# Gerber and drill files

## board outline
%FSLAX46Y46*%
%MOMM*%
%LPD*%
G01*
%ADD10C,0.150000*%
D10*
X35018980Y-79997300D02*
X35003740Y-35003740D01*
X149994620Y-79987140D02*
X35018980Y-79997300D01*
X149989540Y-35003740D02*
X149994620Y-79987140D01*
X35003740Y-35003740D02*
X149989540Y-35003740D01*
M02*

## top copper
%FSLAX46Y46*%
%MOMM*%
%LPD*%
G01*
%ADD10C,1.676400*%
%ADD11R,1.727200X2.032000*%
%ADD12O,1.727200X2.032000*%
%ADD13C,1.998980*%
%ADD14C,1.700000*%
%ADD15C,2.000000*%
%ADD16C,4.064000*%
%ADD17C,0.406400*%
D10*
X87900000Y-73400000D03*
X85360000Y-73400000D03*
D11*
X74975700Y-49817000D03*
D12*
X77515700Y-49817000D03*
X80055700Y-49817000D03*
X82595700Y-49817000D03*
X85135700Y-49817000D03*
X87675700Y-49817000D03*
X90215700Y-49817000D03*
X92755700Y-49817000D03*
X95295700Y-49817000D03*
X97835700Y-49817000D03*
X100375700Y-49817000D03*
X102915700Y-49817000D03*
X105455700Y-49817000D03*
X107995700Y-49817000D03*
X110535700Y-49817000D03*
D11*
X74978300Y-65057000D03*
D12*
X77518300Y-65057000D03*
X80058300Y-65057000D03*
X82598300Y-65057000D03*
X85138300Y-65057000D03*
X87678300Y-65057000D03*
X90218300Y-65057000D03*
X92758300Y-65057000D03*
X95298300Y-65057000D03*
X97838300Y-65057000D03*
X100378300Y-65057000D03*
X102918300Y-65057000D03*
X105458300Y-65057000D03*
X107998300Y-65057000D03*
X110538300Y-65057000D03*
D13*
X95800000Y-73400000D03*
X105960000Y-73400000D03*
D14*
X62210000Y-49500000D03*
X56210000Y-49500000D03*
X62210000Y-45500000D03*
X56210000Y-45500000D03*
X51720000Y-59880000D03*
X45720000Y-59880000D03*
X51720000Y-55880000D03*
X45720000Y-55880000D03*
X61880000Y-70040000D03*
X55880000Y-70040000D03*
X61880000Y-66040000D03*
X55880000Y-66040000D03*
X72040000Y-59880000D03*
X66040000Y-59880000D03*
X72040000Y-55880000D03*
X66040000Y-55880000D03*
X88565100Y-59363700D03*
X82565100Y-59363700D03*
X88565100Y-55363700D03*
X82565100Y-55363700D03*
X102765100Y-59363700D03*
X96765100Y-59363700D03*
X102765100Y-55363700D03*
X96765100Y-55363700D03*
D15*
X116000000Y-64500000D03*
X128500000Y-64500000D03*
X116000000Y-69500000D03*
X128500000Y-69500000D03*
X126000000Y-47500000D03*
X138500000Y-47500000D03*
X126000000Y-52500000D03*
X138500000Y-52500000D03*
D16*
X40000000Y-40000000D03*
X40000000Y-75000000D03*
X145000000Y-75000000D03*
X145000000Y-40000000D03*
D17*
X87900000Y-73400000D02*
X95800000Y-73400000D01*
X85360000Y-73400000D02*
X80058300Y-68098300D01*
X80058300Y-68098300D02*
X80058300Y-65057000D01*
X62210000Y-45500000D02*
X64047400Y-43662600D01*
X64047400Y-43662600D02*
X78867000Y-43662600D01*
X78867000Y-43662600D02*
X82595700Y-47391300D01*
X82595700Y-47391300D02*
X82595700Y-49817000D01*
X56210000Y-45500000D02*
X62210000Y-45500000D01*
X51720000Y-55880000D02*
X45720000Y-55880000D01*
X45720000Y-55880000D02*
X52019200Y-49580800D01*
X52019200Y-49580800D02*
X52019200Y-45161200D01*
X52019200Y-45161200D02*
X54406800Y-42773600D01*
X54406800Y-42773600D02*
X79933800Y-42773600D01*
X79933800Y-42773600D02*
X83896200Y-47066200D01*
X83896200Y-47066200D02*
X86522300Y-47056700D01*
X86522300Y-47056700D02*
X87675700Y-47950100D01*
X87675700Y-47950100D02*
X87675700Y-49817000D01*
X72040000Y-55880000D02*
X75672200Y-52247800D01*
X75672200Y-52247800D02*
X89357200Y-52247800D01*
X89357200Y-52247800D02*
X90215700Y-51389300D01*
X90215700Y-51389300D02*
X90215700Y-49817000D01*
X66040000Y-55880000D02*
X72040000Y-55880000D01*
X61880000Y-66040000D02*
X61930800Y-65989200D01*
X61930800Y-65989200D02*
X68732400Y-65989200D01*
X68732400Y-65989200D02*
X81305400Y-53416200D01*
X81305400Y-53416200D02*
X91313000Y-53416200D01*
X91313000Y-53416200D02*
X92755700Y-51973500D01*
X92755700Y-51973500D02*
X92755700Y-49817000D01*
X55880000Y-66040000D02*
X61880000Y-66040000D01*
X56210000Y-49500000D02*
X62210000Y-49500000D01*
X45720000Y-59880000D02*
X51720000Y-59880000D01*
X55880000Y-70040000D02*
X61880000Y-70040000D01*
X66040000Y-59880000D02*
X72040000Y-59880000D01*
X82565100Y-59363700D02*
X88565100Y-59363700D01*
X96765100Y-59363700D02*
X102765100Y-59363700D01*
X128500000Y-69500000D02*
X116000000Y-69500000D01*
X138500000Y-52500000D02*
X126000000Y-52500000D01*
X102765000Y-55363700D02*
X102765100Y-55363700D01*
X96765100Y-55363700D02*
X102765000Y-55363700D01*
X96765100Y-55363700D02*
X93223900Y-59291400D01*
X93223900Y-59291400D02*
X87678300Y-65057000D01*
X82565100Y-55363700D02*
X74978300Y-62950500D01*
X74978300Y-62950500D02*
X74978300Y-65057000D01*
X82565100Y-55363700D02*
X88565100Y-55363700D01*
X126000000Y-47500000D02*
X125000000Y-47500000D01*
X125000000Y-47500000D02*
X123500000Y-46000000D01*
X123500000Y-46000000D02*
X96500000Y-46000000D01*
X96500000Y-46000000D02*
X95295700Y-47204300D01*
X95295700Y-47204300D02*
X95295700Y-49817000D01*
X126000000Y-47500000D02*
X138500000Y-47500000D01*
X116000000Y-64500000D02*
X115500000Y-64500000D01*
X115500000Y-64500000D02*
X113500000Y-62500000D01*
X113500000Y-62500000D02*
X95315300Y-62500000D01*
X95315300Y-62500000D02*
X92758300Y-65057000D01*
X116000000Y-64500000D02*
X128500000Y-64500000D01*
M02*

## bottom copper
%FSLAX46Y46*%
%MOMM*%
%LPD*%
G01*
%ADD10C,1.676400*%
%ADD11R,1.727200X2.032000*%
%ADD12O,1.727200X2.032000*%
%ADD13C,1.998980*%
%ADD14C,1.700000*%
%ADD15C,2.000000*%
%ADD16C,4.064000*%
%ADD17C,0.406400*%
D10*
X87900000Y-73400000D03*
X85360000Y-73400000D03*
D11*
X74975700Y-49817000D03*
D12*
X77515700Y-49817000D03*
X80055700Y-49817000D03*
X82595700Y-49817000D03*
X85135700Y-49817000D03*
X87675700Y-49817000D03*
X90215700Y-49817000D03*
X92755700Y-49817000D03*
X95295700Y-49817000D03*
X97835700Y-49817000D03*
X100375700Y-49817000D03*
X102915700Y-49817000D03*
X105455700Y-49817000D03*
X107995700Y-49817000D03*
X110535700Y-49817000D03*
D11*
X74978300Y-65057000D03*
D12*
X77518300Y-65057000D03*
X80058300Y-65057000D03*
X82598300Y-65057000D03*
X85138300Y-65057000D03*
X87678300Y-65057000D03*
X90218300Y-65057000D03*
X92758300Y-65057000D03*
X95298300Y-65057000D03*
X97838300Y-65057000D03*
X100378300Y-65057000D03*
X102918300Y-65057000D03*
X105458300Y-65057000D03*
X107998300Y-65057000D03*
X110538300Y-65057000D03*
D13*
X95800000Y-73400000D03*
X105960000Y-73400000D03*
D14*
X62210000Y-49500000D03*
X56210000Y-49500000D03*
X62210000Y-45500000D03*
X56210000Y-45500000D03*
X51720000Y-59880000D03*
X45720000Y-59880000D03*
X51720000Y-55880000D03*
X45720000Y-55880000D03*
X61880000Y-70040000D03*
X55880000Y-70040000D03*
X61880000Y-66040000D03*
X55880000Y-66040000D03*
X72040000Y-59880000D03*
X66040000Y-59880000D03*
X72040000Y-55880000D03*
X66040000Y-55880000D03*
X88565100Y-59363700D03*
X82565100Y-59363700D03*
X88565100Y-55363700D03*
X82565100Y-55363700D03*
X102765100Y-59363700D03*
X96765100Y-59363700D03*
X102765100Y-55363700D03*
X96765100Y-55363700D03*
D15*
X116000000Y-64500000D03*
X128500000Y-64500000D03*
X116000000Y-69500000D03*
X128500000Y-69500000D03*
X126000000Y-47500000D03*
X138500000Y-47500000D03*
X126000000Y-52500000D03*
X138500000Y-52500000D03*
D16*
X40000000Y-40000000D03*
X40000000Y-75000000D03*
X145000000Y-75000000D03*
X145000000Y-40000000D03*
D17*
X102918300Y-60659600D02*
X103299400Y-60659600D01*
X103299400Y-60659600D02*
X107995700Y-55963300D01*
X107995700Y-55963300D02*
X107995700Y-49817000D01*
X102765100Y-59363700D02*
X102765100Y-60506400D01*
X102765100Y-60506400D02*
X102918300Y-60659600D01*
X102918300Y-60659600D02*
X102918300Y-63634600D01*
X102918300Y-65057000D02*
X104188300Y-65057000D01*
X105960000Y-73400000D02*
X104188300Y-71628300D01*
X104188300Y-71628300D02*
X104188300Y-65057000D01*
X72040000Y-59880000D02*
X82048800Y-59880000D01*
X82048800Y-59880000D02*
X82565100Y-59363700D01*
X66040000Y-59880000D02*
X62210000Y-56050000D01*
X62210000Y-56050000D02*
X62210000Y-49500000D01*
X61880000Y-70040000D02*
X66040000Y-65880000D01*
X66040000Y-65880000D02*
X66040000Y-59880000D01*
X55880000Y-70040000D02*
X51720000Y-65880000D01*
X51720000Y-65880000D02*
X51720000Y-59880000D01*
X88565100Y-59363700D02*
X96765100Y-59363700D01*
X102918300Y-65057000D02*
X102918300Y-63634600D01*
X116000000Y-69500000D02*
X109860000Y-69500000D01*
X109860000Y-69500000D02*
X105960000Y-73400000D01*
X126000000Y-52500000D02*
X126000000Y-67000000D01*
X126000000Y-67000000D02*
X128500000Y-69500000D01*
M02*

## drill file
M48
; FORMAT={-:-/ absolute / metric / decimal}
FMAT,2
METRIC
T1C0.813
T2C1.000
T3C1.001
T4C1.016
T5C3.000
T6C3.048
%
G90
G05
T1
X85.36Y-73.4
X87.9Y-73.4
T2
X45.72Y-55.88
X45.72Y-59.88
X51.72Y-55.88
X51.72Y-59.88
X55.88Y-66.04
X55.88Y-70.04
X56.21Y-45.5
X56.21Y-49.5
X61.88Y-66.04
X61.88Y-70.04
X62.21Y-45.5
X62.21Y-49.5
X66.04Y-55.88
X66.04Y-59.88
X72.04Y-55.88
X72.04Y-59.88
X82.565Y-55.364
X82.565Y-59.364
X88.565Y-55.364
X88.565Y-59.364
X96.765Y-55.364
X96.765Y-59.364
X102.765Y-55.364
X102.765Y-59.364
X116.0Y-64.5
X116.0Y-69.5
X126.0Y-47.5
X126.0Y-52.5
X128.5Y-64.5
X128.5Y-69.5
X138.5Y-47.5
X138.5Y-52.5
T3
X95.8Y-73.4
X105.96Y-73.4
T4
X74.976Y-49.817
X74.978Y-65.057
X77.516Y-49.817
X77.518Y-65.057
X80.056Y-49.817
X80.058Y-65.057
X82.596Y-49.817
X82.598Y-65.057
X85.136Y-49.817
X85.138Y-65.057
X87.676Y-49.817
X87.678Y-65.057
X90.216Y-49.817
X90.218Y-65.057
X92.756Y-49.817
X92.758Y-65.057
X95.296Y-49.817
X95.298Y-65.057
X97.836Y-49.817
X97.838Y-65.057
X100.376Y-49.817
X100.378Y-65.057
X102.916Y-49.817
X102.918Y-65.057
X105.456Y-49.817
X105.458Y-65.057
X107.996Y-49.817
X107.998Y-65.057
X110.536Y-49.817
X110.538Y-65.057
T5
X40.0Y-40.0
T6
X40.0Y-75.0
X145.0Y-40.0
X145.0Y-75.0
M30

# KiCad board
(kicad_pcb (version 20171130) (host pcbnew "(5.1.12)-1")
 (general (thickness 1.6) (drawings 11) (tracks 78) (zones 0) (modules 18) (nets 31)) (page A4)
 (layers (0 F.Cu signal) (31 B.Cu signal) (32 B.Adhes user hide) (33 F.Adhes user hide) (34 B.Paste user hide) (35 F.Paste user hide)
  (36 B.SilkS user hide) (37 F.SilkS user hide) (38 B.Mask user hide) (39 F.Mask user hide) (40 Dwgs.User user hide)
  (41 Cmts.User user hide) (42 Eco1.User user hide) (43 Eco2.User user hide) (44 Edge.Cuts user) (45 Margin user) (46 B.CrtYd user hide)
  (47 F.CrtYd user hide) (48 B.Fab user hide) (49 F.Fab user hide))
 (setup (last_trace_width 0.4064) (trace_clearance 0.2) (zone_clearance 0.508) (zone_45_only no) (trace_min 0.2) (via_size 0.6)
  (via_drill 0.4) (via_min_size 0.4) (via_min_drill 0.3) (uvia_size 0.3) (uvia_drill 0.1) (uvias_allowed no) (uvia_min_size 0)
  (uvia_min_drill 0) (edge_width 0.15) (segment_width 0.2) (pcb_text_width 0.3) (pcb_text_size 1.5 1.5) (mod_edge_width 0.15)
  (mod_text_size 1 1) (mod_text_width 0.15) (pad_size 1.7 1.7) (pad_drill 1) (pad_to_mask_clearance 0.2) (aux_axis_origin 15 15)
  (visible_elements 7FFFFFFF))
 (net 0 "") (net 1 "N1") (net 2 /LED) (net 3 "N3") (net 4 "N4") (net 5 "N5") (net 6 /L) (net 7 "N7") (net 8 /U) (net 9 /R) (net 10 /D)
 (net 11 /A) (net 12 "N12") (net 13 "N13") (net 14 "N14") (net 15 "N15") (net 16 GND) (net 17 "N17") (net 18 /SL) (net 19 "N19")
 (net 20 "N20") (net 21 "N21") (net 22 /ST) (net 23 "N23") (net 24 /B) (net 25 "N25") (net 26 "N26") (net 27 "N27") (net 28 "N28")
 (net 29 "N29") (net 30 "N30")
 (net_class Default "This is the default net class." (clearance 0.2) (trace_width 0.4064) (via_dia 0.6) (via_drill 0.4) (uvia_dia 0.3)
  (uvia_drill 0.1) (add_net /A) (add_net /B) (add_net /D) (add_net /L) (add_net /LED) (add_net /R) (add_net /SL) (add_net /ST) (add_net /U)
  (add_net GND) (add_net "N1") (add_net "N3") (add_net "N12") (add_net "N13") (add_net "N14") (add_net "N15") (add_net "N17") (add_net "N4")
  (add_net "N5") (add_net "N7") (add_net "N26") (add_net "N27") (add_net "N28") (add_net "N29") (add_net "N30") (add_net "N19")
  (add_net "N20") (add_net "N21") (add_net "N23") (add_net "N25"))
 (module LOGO (layer B.Cu) (at 92.4306 44.6532)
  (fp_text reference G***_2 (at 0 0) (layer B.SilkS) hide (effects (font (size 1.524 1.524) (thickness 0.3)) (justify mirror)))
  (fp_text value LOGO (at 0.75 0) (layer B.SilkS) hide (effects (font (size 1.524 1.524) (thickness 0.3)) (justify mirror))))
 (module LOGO (layer F.Cu) (at 139.0396 63.246)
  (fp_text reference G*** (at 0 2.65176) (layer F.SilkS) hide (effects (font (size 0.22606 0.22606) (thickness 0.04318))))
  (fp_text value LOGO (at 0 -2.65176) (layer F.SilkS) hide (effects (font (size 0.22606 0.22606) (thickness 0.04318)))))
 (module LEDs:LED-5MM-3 (layer F.Cu) (at 87.9 73.4 180)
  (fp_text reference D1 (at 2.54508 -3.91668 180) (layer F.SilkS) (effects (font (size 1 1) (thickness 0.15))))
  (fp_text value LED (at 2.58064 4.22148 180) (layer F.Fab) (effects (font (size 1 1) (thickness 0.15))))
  (pad 1 thru_hole circle (at 0 0) (size 1.6764 1.6764) (drill 0.8128) (layers *.Cu *.Mask F.SilkS) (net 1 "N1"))
  (pad 2 thru_hole circle (at 2.54 0) (size 1.6764 1.6764) (drill 0.8128) (layers *.Cu *.Mask F.SilkS) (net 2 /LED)))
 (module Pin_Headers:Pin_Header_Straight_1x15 (layer B.Cu) (at 74.9757 49.817 270)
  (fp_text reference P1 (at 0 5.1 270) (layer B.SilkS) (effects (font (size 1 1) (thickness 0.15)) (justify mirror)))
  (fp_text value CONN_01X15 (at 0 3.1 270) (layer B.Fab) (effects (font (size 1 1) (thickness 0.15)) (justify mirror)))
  (pad 1 thru_hole rect (at 0 0 270) (size 2.032 1.7272) (drill 1.016) (layers *.Cu *.Mask B.SilkS) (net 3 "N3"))
  (pad 2 thru_hole oval (at 0 -2.54 270) (size 2.032 1.7272) (drill 1.016) (layers *.Cu *.Mask B.SilkS) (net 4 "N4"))
  (pad 3 thru_hole oval (at 0 -5.08 270) (size 2.032 1.7272) (drill 1.016) (layers *.Cu *.Mask B.SilkS) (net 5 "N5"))
  (pad 4 thru_hole oval (at 0 -7.62 270) (size 2.032 1.7272) (drill 1.016) (layers *.Cu *.Mask B.SilkS) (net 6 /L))
  (pad 5 thru_hole oval (at 0 -10.16 270) (size 2.032 1.7272) (drill 1.016) (layers *.Cu *.Mask B.SilkS) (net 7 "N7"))
  (pad 6 thru_hole oval (at 0 -12.7 270) (size 2.032 1.7272) (drill 1.016) (layers *.Cu *.Mask B.SilkS) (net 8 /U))
  (pad 7 thru_hole oval (at 0 -15.24 270) (size 2.032 1.7272) (drill 1.016) (layers *.Cu *.Mask B.SilkS) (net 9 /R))
  (pad 8 thru_hole oval (at 0 -17.78 270) (size 2.032 1.7272) (drill 1.016) (layers *.Cu *.Mask B.SilkS) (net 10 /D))
  (pad 9 thru_hole oval (at 0 -20.32 270) (size 2.032 1.7272) (drill 1.016) (layers *.Cu *.Mask B.SilkS) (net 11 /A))
  (pad 10 thru_hole oval (at 0 -22.86 270) (size 2.032 1.7272) (drill 1.016) (layers *.Cu *.Mask B.SilkS) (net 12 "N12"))
  (pad 11 thru_hole oval (at 0 -25.4 270) (size 2.032 1.7272) (drill 1.016) (layers *.Cu *.Mask B.SilkS) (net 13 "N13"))
  (pad 12 thru_hole oval (at 0 -27.94 270) (size 2.032 1.7272) (drill 1.016) (layers *.Cu *.Mask B.SilkS) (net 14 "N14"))
  (pad 13 thru_hole oval (at 0 -30.48 270) (size 2.032 1.7272) (drill 1.016) (layers *.Cu *.Mask B.SilkS) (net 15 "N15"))
  (pad 14 thru_hole oval (at 0 -33.02 270) (size 2.032 1.7272) (drill 1.016) (layers *.Cu *.Mask B.SilkS) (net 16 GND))
  (pad 15 thru_hole oval (at 0 -35.56 270) (size 2.032 1.7272) (drill 1.016) (layers *.Cu *.Mask B.SilkS) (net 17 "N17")))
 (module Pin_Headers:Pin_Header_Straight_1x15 (layer B.Cu) (at 74.9783 65.057 270)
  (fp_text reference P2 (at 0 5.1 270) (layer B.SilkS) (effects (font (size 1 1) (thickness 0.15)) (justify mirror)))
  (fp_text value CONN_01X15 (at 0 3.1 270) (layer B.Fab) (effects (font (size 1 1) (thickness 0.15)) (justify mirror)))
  (pad 1 thru_hole rect (at 0 0 270) (size 2.032 1.7272) (drill 1.016) (layers *.Cu *.Mask B.SilkS) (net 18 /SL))
  (pad 2 thru_hole oval (at 0 -2.54 270) (size 2.032 1.7272) (drill 1.016) (layers *.Cu *.Mask B.SilkS) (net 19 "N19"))
  (pad 3 thru_hole oval (at 0 -5.08 270) (size 2.032 1.7272) (drill 1.016) (layers *.Cu *.Mask B.SilkS) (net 2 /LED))
  (pad 4 thru_hole oval (at 0 -7.62 270) (size 2.032 1.7272) (drill 1.016) (layers *.Cu *.Mask B.SilkS) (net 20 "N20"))
  (pad 5 thru_hole oval (at 0 -10.16 270) (size 2.032 1.7272) (drill 1.016) (layers *.Cu *.Mask B.SilkS) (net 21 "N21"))
  (pad 6 thru_hole oval (at 0 -12.7 270) (size 2.032 1.7272) (drill 1.016) (layers *.Cu *.Mask B.SilkS) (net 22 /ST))
  (pad 7 thru_hole oval (at 0 -15.24 270) (size 2.032 1.7272) (drill 1.016) (layers *.Cu *.Mask B.SilkS) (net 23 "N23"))
  (pad 8 thru_hole oval (at 0 -17.78 270) (size 2.032 1.7272) (drill 1.016) (layers *.Cu *.Mask B.SilkS) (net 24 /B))
  (pad 9 thru_hole oval (at 0 -20.32 270) (size 2.032 1.7272) (drill 1.016) (layers *.Cu *.Mask B.SilkS) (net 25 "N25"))
  (pad 10 thru_hole oval (at 0 -22.86 270) (size 2.032 1.7272) (drill 1.016) (layers *.Cu *.Mask B.SilkS) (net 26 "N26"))
  (pad 11 thru_hole oval (at 0 -25.4 270) (size 2.032 1.7272) (drill 1.016) (layers *.Cu *.Mask B.SilkS) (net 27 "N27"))
  (pad 12 thru_hole oval (at 0 -27.94 270) (size 2.032 1.7272) (drill 1.016) (layers *.Cu *.Mask B.SilkS) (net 16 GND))
  (pad 13 thru_hole oval (at 0 -30.48 270) (size 2.032 1.7272) (drill 1.016) (layers *.Cu *.Mask B.SilkS) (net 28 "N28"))
  (pad 14 thru_hole oval (at 0 -33.02 270) (size 2.032 1.7272) (drill 1.016) (layers *.Cu *.Mask B.SilkS) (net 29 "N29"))
  (pad 15 thru_hole oval (at 0 -35.56 270) (size 2.032 1.7272) (drill 1.016) (layers *.Cu *.Mask B.SilkS) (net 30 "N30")))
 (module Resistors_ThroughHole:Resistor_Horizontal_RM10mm (layer F.Cu) (at 95.8 73.4)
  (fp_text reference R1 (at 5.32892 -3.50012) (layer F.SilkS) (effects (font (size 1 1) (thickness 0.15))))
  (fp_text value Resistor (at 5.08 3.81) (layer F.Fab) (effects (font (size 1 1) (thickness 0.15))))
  (pad 1 thru_hole circle (at 0 0) (size 1.99898 1.99898) (drill 1.00076) (layers *.Cu *.SilkS *.Mask) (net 1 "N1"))
  (pad 2 thru_hole circle (at 10.16 0) (size 1.99898 1.99898) (drill 1.00076) (layers *.Cu *.SilkS *.Mask) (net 16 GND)))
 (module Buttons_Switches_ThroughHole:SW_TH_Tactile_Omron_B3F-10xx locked (layer F.Cu) (at 56.21 45.5)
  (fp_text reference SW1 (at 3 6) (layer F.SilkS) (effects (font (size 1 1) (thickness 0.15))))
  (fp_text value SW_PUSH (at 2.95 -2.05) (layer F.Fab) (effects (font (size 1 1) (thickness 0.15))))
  (pad 4 thru_hole circle (at 6 4) (size 1.7 1.7) (drill 1) (layers *.Cu *.Mask) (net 16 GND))
  (pad 3 thru_hole circle (at 0 4) (size 1.7 1.7) (drill 1) (layers *.Cu *.Mask) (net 16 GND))
  (pad 1 thru_hole circle (at 6 0) (size 1.7 1.7) (drill 1) (layers *.Cu *.Mask) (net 6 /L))
  (pad 1 thru_hole circle (at 0 0) (size 1.7 1.7) (drill 1) (layers *.Cu *.Mask) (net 6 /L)))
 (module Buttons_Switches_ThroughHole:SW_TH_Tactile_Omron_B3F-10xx (layer F.Cu) (at 45.72 55.88)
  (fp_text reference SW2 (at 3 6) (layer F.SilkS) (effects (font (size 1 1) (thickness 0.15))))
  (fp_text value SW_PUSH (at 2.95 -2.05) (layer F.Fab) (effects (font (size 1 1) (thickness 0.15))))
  (pad 4 thru_hole circle (at 6 4) (size 1.7 1.7) (drill 1) (layers *.Cu *.Mask) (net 16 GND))
  (pad 3 thru_hole circle (at 0 4) (size 1.7 1.7) (drill 1) (layers *.Cu *.Mask) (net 16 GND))
  (pad 1 thru_hole circle (at 6 0) (size 1.7 1.7) (drill 1) (layers *.Cu *.Mask) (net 8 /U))
  (pad 1 thru_hole circle (at 0 0) (size 1.7 1.7) (drill 1) (layers *.Cu *.Mask) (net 8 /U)))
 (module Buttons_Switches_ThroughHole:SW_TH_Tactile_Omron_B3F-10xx (layer F.Cu) (at 55.88 66.04)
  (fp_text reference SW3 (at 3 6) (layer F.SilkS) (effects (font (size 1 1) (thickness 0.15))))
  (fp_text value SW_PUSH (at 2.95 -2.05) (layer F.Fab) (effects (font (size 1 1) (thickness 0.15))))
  (pad 4 thru_hole circle (at 6 4) (size 1.7 1.7) (drill 1) (layers *.Cu *.Mask) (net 16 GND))
  (pad 3 thru_hole circle (at 0 4) (size 1.7 1.7) (drill 1) (layers *.Cu *.Mask) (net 16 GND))
  (pad 2 thru_hole circle (at 6 0) (size 1.7 1.7) (drill 1) (layers *.Cu *.Mask) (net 10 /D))
  (pad 1 thru_hole circle (at 0 0) (size 1.7 1.7) (drill 1) (layers *.Cu *.Mask) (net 10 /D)))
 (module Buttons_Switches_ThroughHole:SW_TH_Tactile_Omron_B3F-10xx (layer F.Cu) (at 66.04 55.88)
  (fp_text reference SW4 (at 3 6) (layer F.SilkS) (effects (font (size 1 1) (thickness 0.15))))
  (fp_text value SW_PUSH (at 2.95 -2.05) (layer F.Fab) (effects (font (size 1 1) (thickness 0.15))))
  (pad 4 thru_hole circle (at 6 4) (size 1.7 1.7) (drill 1) (layers *.Cu *.Mask) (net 16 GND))
  (pad 3 thru_hole circle (at 0 4) (size 1.7 1.7) (drill 1) (layers *.Cu *.Mask) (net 16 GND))
  (pad 2 thru_hole circle (at 6 0) (size 1.7 1.7) (drill 1) (layers *.Cu *.Mask) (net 9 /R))
  (pad 1 thru_hole circle (at 0 0) (size 1.7 1.7) (drill 1) (layers *.Cu *.Mask) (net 9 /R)))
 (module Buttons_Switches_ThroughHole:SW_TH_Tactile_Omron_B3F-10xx (layer F.Cu) (at 82.5651 55.3637)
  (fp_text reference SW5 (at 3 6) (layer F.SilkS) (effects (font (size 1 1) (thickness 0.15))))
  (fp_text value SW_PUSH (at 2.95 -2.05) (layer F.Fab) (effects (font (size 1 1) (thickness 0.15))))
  (pad 4 thru_hole circle (at 6 4) (size 1.7 1.7) (drill 1) (layers *.Cu *.Mask) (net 16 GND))
  (pad 3 thru_hole circle (at 0 4) (size 1.7 1.7) (drill 1) (layers *.Cu *.Mask) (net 16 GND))
  (pad 2 thru_hole circle (at 6 0) (size 1.7 1.7) (drill 1) (layers *.Cu *.Mask) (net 18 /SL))
  (pad 1 thru_hole circle (at 0 0) (size 1.7 1.7) (drill 1) (layers *.Cu *.Mask) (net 18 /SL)))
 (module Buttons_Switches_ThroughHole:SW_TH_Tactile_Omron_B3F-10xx (layer F.Cu) (at 96.7651 55.3637)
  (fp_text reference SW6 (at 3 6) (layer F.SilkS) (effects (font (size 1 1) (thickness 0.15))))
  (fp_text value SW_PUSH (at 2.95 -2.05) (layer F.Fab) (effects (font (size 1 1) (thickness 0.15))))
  (pad 4 thru_hole circle (at 6 4) (size 1.7 1.7) (drill 1) (layers *.Cu *.Mask) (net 16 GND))
  (pad 3 thru_hole circle (at 0 4) (size 1.7 1.7) (drill 1) (layers *.Cu *.Mask) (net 16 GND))
  (pad 2 thru_hole circle (at 6 0) (size 1.7 1.7) (drill 1) (layers *.Cu *.Mask) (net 22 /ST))
  (pad 1 thru_hole circle (at 0 0) (size 1.7 1.7) (drill 1) (layers *.Cu *.Mask) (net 22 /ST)))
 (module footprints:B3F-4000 (layer F.Cu) (at 116 64.5)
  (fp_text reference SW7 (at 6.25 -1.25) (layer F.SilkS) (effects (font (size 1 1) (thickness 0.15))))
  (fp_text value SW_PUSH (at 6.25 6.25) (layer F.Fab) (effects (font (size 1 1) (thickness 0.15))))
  (pad 1 thru_hole circle (at 0 0) (size 2 2) (drill 1) (layers *.Cu *.Mask F.SilkS) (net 24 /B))
  (pad 1 thru_hole circle (at 12.5 0) (size 2 2) (drill 1) (layers *.Cu *.Mask F.SilkS) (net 24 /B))
  (pad 2 thru_hole circle (at 0 5) (size 2 2) (drill 1) (layers *.Cu *.Mask F.SilkS) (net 16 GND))
  (pad 2 thru_hole circle (at 12.5 5) (size 2 2) (drill 1) (layers *.Cu *.Mask F.SilkS) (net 16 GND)))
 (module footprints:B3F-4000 (layer F.Cu) (at 126 47.5)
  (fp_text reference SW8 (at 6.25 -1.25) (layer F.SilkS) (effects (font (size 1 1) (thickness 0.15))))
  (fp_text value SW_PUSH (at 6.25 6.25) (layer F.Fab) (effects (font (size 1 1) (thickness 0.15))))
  (pad 1 thru_hole circle (at 0 0) (size 2 2) (drill 1) (layers *.Cu *.Mask F.SilkS) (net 11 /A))
  (pad 1 thru_hole circle (at 12.5 0) (size 2 2) (drill 1) (layers *.Cu *.Mask F.SilkS) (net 11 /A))
  (pad 2 thru_hole circle (at 0 5) (size 2 2) (drill 1) (layers *.Cu *.Mask F.SilkS) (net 16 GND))
  (pad 2 thru_hole circle (at 12.5 5) (size 2 2) (drill 1) (layers *.Cu *.Mask F.SilkS) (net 16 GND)))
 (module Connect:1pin (layer F.Cu) (at 40 40)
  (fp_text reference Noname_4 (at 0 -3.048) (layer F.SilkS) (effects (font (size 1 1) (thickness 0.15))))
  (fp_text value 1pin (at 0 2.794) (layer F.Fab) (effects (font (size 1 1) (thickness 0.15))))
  (pad "" np_thru_hole circle (at 0 0) (size 4.064 4.064) (drill 3) (layers *.Cu *.Mask F.SilkS)))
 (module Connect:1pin (layer F.Cu) (at 40 75)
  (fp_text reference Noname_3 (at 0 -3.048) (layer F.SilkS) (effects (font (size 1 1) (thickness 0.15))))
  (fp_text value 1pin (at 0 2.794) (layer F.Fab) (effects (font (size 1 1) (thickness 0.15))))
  (pad "" np_thru_hole circle (at 0 0) (size 4.064 4.064) (drill 3.048) (layers *.Cu *.Mask F.SilkS)))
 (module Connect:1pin (layer F.Cu) (at 145 75)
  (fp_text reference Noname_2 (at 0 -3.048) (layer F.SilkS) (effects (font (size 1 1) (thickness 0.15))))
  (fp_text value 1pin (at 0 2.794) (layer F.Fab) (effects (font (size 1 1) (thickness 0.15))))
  (pad "" np_thru_hole circle (at 0 0) (size 4.064 4.064) (drill 3.048) (layers *.Cu *.Mask F.SilkS)))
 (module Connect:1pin (layer F.Cu) (at 145 40)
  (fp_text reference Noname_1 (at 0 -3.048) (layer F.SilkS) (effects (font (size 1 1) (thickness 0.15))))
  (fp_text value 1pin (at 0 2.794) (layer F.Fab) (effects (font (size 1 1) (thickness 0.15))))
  (pad "" np_thru_hole circle (at 0 0) (size 4.064 4.064) (drill 3.048) (layers *.Cu *.Mask F.SilkS)))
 (gr_line (start 35.01898 79.9973) (end 35.00374 35.00374) (layer Edge.Cuts) (width 0.15))
 (gr_line (start 149.99462 79.98714) (end 35.01898 79.9973) (layer Edge.Cuts) (width 0.15))
 (gr_line (start 149.98954 35.00374) (end 149.99462 79.98714) (layer Edge.Cuts) (width 0.15))
 (gr_line (start 35.00374 35.00374) (end 149.98954 35.00374) (layer Edge.Cuts) (width 0.15))
 (segment (start 87.9 73.4) (end 95.8 73.4) (width 0.4064) (layer F.Cu) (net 1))
 (segment (start 85.36 73.4) (end 80.0583 68.0983) (width 0.4064) (layer F.Cu) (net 2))
 (segment (start 80.0583 68.0983) (end 80.0583 65.057) (width 0.4064) (layer F.Cu) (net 2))
 (segment (start 62.21 45.5) (end 64.0474 43.6626) (width 0.4064) (layer F.Cu) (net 6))
 (segment (start 64.0474 43.6626) (end 78.867 43.6626) (width 0.4064) (layer F.Cu) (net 6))
 (segment (start 78.867 43.6626) (end 82.5957 47.3913) (width 0.4064) (layer F.Cu) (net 6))
 (segment (start 82.5957 47.3913) (end 82.5957 49.817) (width 0.4064) (layer F.Cu) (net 6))
 (segment (start 56.21 45.5) (end 62.21 45.5) (width 0.4064) (layer F.Cu) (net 6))
 (segment (start 51.72 55.88) (end 45.72 55.88) (width 0.4064) (layer F.Cu) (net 8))
 (segment (start 45.72 55.88) (end 52.0192 49.5808) (width 0.4064) (layer F.Cu) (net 8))
 (segment (start 52.0192 49.5808) (end 52.0192 45.1612) (width 0.4064) (layer F.Cu) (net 8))
 (segment (start 52.0192 45.1612) (end 54.4068 42.7736) (width 0.4064) (layer F.Cu) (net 8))
 (segment (start 54.4068 42.7736) (end 79.9338 42.7736) (width 0.4064) (layer F.Cu) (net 8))
 (segment (start 79.9338 42.7736) (end 83.8962 47.0662) (width 0.4064) (layer F.Cu) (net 8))
 (segment (start 83.8962 47.0662) (end 86.5223 47.0567) (width 0.4064) (layer F.Cu) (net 8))
 (segment (start 86.5223 47.0567) (end 87.6757 47.9501) (width 0.4064) (layer F.Cu) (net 8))
 (segment (start 87.6757 47.9501) (end 87.6757 49.817) (width 0.4064) (layer F.Cu) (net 8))
 (segment (start 72.04 55.88) (end 75.6722 52.2478) (width 0.4064) (layer F.Cu) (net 9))
 (segment (start 75.6722 52.2478) (end 89.3572 52.2478) (width 0.4064) (layer F.Cu) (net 9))
 (segment (start 89.3572 52.2478) (end 90.2157 51.3893) (width 0.4064) (layer F.Cu) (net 9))
 (segment (start 90.2157 51.3893) (end 90.2157 49.817) (width 0.4064) (layer F.Cu) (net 9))
 (segment (start 66.04 55.88) (end 72.04 55.88) (width 0.4064) (layer F.Cu) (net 9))
 (segment (start 61.88 66.04) (end 61.9308 65.9892) (width 0.4064) (layer F.Cu) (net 10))
 (segment (start 61.9308 65.9892) (end 68.7324 65.9892) (width 0.4064) (layer F.Cu) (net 10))
 (segment (start 68.7324 65.9892) (end 81.3054 53.4162) (width 0.4064) (layer F.Cu) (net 10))
 (segment (start 81.3054 53.4162) (end 91.313 53.4162) (width 0.4064) (layer F.Cu) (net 10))
 (segment (start 91.313 53.4162) (end 92.7557 51.9735) (width 0.4064) (layer F.Cu) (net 10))
 (segment (start 92.7557 51.9735) (end 92.7557 49.817) (width 0.4064) (layer F.Cu) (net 10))
 (segment (start 55.88 66.04) (end 61.88 66.04) (width 0.4064) (layer F.Cu) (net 10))
 (segment (start 102.9183 60.6596) (end 103.2994 60.6596) (width 0.4064) (layer B.Cu) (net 16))
 (segment (start 103.2994 60.6596) (end 107.9957 55.9633) (width 0.4064) (layer B.Cu) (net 16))
 (segment (start 107.9957 55.9633) (end 107.9957 49.817) (width 0.4064) (layer B.Cu) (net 16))
 (segment (start 102.7651 59.3637) (end 102.7651 60.5064) (width 0.4064) (layer B.Cu) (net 16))
 (segment (start 102.7651 60.5064) (end 102.9183 60.6596) (width 0.4064) (layer B.Cu) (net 16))
 (segment (start 102.9183 60.6596) (end 102.9183 63.6346) (width 0.4064) (layer B.Cu) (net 16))
 (segment (start 102.9183 65.057) (end 104.1883 65.057) (width 0.4064) (layer B.Cu) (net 16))
 (segment (start 105.96 73.4) (end 104.1883 71.6283) (width 0.4064) (layer B.Cu) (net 16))
 (segment (start 104.1883 71.6283) (end 104.1883 65.057) (width 0.4064) (layer B.Cu) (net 16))
 (segment (start 72.04 59.88) (end 82.0488 59.88) (width 0.4064) (layer B.Cu) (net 16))
 (segment (start 82.0488 59.88) (end 82.5651 59.3637) (width 0.4064) (layer B.Cu) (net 16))
 (segment (start 56.21 49.5) (end 62.21 49.5) (width 0.4064) (layer F.Cu) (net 16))
 (segment (start 66.04 59.88) (end 62.21 56.05) (width 0.4064) (layer B.Cu) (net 16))
 (segment (start 62.21 56.05) (end 62.21 49.5) (width 0.4064) (layer B.Cu) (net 16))
 (segment (start 61.88 70.04) (end 66.04 65.88) (width 0.4064) (layer B.Cu) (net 16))
 (segment (start 66.04 65.88) (end 66.04 59.88) (width 0.4064) (layer B.Cu) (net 16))
 (segment (start 45.72 59.88) (end 51.72 59.88) (width 0.4064) (layer F.Cu) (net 16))
 (segment (start 55.88 70.04) (end 51.72 65.88) (width 0.4064) (layer B.Cu) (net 16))
 (segment (start 51.72 65.88) (end 51.72 59.88) (width 0.4064) (layer B.Cu) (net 16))
 (segment (start 55.88 70.04) (end 61.88 70.04) (width 0.4064) (layer F.Cu) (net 16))
 (segment (start 66.04 59.88) (end 72.04 59.88) (width 0.4064) (layer F.Cu) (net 16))
 (segment (start 88.5651 59.3637) (end 96.7651 59.3637) (width 0.4064) (layer B.Cu) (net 16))
 (segment (start 82.5651 59.3637) (end 88.5651 59.3637) (width 0.4064) (layer F.Cu) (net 16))
 (segment (start 102.9183 65.057) (end 102.9183 63.6346) (width 0.4064) (layer B.Cu) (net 16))
 (segment (start 96.7651 59.3637) (end 102.7651 59.3637) (width 0.4064) (layer F.Cu) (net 16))
 (segment (start 116 69.5) (end 109.86 69.5) (width 0.4064) (layer B.Cu) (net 16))
 (segment (start 109.86 69.5) (end 105.96 73.4) (width 0.4064) (layer B.Cu) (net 16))
 (segment (start 128.5 69.5) (end 116 69.5) (width 0.4064) (layer F.Cu) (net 16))
 (segment (start 126 52.5) (end 126 67) (width 0.4064) (layer B.Cu) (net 16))
 (segment (start 126 67) (end 128.5 69.5) (width 0.4064) (layer B.Cu) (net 16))
 (segment (start 138.5 52.5) (end 126 52.5) (width 0.4064) (layer F.Cu) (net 16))
 (segment (start 102.765 55.3637) (end 102.7651 55.3637) (width 0.4064) (layer F.Cu) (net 22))
 (segment (start 96.7651 55.3637) (end 102.765 55.3637) (width 0.4064) (layer F.Cu) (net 22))
 (segment (start 96.7651 55.3637) (end 93.2239 59.2914) (width 0.4064) (layer F.Cu) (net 22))
 (segment (start 93.2239 59.2914) (end 87.6783 65.057) (width 0.4064) (layer F.Cu) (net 22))
 (segment (start 82.5651 55.3637) (end 74.9783 62.9505) (width 0.4064) (layer F.Cu) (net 18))
 (segment (start 74.9783 62.9505) (end 74.9783 65.057) (width 0.4064) (layer F.Cu) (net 18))
 (segment (start 82.5651 55.3637) (end 88.5651 55.3637) (width 0.4064) (layer F.Cu) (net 18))
 (segment (start 126 47.5) (end 125 47.5) (width 0.4064) (layer F.Cu) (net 11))
 (segment (start 125 47.5) (end 123.5 46) (width 0.4064) (layer F.Cu) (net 11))
 (segment (start 123.5 46) (end 96.5 46) (width 0.4064) (layer F.Cu) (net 11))
 (segment (start 96.5 46) (end 95.2957 47.2043) (width 0.4064) (layer F.Cu) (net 11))
 (segment (start 95.2957 47.2043) (end 95.2957 49.817) (width 0.4064) (layer F.Cu) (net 11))
 (segment (start 126 47.5) (end 138.5 47.5) (width 0.4064) (layer F.Cu) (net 11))
 (segment (start 116 64.5) (end 115.5 64.5) (width 0.4064) (layer F.Cu) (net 24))
 (segment (start 115.5 64.5) (end 113.5 62.5) (width 0.4064) (layer F.Cu) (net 24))
 (segment (start 113.5 62.5) (end 95.3153 62.5) (width 0.4064) (layer F.Cu) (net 24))
 (segment (start 95.3153 62.5) (end 92.7583 65.057) (width 0.4064) (layer F.Cu) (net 24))
 (segment (start 116 64.5) (end 128.5 64.5) (width 0.4064) (layer F.Cu) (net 24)))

